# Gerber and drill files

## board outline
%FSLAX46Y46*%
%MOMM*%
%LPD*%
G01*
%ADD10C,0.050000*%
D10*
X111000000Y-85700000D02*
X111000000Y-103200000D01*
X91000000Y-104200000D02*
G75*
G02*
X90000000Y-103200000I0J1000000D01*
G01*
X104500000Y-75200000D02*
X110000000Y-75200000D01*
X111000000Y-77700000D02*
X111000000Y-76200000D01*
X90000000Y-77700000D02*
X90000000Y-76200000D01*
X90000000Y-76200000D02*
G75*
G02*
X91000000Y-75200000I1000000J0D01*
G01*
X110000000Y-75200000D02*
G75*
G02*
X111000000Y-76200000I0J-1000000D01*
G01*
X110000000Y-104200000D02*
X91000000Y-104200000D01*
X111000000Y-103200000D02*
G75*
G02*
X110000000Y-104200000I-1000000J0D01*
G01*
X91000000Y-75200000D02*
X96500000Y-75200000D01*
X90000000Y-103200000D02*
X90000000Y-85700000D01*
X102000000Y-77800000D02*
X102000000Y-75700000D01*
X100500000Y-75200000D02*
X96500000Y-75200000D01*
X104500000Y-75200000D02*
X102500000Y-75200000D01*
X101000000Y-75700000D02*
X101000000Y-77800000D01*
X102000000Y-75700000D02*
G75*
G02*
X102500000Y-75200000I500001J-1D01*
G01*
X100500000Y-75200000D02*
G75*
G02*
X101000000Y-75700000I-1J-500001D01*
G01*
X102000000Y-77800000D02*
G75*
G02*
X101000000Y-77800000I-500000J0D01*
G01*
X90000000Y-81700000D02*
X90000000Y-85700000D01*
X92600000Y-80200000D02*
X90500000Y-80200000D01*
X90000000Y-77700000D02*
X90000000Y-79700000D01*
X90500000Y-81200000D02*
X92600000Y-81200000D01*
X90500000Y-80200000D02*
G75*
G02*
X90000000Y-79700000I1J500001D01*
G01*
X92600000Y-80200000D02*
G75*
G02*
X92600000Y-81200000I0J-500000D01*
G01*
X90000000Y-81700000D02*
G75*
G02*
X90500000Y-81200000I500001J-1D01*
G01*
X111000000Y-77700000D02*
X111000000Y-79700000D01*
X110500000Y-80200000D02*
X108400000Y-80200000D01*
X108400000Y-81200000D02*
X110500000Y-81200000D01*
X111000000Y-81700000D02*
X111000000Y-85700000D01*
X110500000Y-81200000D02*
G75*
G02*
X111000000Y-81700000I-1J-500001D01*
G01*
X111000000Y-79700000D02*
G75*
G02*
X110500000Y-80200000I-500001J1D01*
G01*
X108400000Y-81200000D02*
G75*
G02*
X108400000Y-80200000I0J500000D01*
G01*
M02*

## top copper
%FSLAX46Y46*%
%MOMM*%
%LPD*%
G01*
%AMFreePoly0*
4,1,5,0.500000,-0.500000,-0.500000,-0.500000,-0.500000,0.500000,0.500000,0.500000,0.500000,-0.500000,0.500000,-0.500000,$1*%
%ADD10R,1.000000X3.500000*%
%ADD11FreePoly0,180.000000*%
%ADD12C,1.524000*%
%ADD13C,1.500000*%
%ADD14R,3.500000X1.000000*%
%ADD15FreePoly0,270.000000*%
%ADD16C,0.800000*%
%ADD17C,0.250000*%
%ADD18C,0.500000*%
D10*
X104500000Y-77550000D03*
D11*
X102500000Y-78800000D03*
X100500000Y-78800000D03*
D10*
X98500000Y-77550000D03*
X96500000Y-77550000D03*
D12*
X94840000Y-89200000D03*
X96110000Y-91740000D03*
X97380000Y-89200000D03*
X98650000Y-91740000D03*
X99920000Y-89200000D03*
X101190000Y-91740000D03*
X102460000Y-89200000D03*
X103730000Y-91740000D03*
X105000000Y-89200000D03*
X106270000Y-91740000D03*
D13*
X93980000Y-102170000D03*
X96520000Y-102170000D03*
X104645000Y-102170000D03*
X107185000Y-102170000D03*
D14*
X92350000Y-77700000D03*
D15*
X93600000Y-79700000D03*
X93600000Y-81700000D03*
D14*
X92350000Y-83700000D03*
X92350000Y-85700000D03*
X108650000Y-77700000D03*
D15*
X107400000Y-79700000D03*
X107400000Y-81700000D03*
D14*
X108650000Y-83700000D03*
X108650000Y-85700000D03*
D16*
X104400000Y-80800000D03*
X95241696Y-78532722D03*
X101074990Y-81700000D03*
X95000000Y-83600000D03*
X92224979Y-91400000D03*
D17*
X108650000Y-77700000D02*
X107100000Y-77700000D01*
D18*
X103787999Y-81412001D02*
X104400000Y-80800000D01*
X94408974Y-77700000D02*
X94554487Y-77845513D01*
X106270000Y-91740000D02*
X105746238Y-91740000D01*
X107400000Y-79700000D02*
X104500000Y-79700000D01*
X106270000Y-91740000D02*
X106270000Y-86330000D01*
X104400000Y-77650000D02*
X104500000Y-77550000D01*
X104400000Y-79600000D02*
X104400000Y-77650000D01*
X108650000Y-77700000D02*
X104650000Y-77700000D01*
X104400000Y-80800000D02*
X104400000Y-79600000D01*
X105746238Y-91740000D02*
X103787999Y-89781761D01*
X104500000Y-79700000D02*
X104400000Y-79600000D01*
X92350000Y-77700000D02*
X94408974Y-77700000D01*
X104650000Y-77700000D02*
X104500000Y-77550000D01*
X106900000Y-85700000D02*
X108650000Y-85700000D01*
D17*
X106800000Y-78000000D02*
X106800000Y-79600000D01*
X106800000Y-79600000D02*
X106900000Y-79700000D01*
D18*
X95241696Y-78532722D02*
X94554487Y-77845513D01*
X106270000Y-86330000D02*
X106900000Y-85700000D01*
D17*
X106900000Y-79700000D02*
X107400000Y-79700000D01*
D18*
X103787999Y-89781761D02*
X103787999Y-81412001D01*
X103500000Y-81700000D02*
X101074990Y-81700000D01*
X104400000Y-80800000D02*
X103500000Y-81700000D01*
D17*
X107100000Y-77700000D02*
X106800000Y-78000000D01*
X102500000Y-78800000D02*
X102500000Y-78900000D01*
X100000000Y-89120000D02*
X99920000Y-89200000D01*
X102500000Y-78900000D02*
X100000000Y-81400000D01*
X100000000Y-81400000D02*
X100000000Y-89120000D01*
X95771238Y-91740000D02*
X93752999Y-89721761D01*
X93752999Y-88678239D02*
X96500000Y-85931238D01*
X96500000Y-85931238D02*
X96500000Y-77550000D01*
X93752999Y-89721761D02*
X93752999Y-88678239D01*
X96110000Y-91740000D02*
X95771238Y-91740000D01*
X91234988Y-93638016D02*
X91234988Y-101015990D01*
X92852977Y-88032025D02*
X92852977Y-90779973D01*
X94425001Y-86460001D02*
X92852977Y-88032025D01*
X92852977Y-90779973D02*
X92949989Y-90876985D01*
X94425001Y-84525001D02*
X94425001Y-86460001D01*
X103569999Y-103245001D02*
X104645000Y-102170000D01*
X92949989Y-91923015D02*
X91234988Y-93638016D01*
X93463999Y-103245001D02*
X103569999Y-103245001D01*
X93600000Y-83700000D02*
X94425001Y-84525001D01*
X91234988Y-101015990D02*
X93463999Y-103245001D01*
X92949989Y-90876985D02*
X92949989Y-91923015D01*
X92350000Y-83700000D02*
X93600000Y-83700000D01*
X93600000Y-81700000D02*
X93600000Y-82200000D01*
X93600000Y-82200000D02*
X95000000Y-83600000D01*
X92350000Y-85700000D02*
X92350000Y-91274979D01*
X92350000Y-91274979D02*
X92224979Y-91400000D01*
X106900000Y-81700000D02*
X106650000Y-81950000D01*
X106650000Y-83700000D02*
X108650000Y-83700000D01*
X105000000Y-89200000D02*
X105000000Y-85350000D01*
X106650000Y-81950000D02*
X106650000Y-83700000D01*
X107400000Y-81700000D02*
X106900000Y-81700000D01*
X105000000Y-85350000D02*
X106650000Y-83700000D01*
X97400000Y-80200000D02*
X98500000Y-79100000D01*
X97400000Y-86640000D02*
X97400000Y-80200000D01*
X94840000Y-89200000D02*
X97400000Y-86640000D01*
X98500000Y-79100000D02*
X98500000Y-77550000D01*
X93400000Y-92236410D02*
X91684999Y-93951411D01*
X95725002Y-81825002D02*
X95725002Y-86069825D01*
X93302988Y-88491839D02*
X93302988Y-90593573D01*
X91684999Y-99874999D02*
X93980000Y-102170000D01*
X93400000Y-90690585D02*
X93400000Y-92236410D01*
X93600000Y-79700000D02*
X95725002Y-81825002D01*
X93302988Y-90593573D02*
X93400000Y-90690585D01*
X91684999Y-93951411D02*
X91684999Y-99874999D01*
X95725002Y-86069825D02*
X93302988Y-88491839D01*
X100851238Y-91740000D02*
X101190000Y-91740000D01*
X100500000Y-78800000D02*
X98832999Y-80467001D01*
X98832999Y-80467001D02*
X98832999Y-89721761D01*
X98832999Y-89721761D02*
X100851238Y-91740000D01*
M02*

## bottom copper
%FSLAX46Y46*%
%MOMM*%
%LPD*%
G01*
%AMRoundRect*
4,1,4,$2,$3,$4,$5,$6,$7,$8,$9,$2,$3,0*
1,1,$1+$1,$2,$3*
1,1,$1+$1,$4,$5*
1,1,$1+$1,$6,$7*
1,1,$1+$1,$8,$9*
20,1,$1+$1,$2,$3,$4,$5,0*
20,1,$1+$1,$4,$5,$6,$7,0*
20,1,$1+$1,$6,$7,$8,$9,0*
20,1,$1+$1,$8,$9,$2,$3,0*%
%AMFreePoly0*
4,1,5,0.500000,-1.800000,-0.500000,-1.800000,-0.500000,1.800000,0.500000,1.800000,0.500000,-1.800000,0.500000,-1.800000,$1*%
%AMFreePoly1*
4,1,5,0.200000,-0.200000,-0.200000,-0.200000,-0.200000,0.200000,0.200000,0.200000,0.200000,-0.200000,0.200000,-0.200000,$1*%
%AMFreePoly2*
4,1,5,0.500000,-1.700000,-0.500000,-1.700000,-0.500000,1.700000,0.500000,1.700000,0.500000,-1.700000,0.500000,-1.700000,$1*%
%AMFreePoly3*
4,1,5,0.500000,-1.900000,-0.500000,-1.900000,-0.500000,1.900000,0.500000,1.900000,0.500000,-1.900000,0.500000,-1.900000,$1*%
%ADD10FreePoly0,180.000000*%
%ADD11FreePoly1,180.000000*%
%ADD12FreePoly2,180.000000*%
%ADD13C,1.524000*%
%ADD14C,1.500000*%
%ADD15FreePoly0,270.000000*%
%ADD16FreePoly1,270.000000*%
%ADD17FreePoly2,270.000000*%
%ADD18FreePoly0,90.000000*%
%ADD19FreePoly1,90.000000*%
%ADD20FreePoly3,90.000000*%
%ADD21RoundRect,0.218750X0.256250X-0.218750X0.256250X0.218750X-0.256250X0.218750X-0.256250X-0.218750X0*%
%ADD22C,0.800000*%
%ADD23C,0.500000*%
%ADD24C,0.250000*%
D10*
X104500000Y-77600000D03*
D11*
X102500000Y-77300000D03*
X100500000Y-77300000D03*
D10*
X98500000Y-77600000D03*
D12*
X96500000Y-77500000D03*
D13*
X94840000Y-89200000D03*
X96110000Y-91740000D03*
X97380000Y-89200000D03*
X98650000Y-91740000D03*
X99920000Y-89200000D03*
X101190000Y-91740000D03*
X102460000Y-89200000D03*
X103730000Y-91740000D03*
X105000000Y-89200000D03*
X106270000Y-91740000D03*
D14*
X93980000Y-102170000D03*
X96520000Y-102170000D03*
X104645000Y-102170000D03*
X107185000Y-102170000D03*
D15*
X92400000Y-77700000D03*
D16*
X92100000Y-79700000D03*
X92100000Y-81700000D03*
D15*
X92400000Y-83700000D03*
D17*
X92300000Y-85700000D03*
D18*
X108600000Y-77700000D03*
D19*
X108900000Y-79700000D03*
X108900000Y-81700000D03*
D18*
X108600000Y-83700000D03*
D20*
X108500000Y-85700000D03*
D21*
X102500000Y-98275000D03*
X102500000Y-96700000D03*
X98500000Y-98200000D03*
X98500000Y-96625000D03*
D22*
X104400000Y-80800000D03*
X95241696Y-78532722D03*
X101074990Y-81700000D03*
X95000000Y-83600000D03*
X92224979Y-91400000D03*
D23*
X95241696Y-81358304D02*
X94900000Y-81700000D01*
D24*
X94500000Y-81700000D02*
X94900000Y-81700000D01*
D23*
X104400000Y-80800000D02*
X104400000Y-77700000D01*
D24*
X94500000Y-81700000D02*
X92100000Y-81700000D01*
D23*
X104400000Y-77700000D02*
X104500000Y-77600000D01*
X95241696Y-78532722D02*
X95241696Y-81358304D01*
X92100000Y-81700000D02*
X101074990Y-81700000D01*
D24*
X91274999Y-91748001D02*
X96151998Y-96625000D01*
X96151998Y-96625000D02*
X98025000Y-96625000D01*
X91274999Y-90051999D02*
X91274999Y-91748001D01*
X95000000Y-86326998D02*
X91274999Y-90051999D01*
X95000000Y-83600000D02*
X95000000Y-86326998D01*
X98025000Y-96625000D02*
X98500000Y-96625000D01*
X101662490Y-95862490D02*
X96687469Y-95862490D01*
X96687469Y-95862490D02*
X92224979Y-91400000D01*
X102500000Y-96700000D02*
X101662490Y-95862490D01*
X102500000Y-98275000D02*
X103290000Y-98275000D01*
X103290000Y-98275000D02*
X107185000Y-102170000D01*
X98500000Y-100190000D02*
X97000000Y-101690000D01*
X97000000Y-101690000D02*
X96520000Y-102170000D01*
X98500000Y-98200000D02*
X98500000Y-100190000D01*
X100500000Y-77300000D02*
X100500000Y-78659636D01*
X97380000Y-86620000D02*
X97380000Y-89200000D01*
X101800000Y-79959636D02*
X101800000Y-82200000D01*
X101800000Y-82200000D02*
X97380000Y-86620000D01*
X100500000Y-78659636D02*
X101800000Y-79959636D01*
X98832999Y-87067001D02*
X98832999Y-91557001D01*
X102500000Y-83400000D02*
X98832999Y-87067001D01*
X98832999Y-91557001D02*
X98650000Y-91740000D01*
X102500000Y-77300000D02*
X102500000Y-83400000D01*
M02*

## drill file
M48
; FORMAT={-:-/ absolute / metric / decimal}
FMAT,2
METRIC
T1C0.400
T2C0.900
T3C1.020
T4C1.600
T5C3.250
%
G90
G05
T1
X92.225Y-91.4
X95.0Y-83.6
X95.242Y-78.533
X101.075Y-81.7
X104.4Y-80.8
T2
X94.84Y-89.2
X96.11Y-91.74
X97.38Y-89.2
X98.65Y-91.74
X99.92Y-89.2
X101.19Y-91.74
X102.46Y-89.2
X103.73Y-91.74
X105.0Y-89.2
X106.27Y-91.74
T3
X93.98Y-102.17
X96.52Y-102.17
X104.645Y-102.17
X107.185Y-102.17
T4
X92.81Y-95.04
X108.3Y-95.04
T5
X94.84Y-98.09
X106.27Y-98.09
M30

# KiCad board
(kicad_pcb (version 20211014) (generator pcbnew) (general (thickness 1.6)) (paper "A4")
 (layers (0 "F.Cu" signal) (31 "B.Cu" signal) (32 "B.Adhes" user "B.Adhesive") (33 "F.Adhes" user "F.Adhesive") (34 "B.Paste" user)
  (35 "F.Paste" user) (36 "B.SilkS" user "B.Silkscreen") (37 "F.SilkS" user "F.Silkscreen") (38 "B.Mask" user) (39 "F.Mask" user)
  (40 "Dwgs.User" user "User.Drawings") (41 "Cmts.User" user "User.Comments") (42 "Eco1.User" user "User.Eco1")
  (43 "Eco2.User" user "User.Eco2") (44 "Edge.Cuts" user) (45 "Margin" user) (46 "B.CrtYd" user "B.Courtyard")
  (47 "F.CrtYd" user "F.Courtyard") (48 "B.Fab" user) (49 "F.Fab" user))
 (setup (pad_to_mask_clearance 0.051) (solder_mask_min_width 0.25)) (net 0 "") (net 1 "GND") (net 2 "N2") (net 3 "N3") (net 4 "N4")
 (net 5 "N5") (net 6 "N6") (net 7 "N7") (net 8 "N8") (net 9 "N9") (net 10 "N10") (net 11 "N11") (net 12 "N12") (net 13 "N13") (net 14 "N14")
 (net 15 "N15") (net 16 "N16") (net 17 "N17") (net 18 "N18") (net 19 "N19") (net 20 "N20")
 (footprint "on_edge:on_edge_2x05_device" (layer "F.Cu") (at 100.5 75.2 180)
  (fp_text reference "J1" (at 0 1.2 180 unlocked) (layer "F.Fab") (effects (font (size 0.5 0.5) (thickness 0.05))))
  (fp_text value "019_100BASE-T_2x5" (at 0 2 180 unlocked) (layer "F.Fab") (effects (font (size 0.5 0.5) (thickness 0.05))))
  (fp_line (start -1.5 -2.6) (end -1.5 -0.5) (layer "Edge.Cuts") (width 0.05))
  (fp_line (start 0 0) (end 4 0) (layer "Edge.Cuts") (width 0.05))
  (fp_line (start -4 0) (end -2 0) (layer "Edge.Cuts") (width 0.05))
  (fp_line (start -0.5 -0.5) (end -0.5 -2.6) (layer "Edge.Cuts") (width 0.05))
  (fp_arc (start -1.5 -0.5) (mid -1.646447 -0.146447) (end -2 0) (layer "Edge.Cuts") (width 0.05))
  (fp_arc (start 0 0) (mid -0.353553 -0.146447) (end -0.5 -0.5) (layer "Edge.Cuts") (width 0.05))
  (fp_arc (start -1.5 -2.6) (mid -1 -3.1) (end -0.5 -2.6) (layer "Edge.Cuts") (width 0.05))
  (pad "1" smd rect locked (at -4 -2.35) (size 1 3.5) (layers "F.Cu" "F.Mask") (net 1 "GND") (zone_connect 0))
  (pad "2" smd custom locked (at -2 -3.6 180) (size 1 1) (layers "F.Cu" "F.Mask") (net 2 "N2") (zone_connect 0)
   (options (clearance outline) (anchor rect)) (primitives))
  (pad "3" smd custom locked (at 0 -3.6 180) (size 1 1) (layers "F.Cu" "F.Mask") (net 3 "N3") (zone_connect 0)
   (options (clearance outline) (anchor rect)) (primitives))
  (pad "4" smd rect locked (at 2 -2.35) (size 1 3.5) (layers "F.Cu" "F.Mask") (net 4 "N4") (zone_connect 0))
  (pad "5" smd rect locked (at 4 -2.35) (size 1 3.5) (layers "F.Cu" "F.Mask") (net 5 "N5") (zone_connect 0))
  (pad "6" smd custom locked (at -4 -2.4 180) (size 1 3.6) (layers "B.Cu" "B.Mask") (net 1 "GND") (zone_connect 0)
   (options (clearance outline) (anchor rect)) (primitives))
  (pad "7" smd custom locked (at -2 -2.1 180) (size 0.4 0.4) (layers "B.Cu" "B.Mask") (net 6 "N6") (zone_connect 0)
   (options (clearance outline) (anchor rect)) (primitives))
  (pad "8" smd custom locked (at 0 -2.1 180) (size 0.4 0.4) (layers "B.Cu" "B.Mask") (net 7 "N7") (zone_connect 0)
   (options (clearance outline) (anchor rect)) (primitives))
  (pad "9" smd custom locked (at 2 -2.4 180) (size 1 3.6) (layers "B.Cu" "B.Mask") (zone_connect 0)
   (options (clearance outline) (anchor rect)) (primitives))
  (pad "10" smd custom locked (at 4 -2.3 180) (size 1 3.4) (layers "B.Cu" "B.Mask") (zone_connect 0)
   (options (clearance outline) (anchor rect)) (primitives)))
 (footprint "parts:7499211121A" (layer "F.Cu") (at 105 89.2 180)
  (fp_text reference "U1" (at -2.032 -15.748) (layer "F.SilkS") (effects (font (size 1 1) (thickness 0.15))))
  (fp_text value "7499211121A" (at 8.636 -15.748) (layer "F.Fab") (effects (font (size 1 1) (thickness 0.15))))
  (pad "" np_thru_hole circle (at -3.3 -5.84 180) (size 1.6 1.6) (drill 1.6) (layers *.Cu *.Mask))
  (pad "" np_thru_hole circle (at 10.16 -8.89 180) (size 3.25 3.25) (drill 3.25) (layers *.Cu *.Mask))
  (pad "" np_thru_hole circle (at 12.19 -5.84 180) (size 1.6 1.6) (drill 1.6) (layers *.Cu *.Mask))
  (pad "" np_thru_hole circle (at -1.27 -8.89 180) (size 3.25 3.25) (drill 3.25) (layers *.Cu *.Mask))
  (pad "1" thru_hole circle (at 10.16 0 180) (size 1.524 1.524) (drill 0.9) (layers *.Cu *.Mask) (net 4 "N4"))
  (pad "2" thru_hole circle (at 8.89 -2.54 180) (size 1.524 1.524) (drill 0.9) (layers *.Cu *.Mask) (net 5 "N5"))
  (pad "3" thru_hole circle (at 7.62 0 180) (size 1.524 1.524) (drill 0.9) (layers *.Cu *.Mask) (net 7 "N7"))
  (pad "4" thru_hole circle (at 6.35 -2.54 180) (size 1.524 1.524) (drill 0.9) (layers *.Cu *.Mask) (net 6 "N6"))
  (pad "5" thru_hole circle (at 5.08 0 180) (size 1.524 1.524) (drill 0.9) (layers *.Cu *.Mask) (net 2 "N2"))
  (pad "6" thru_hole circle (at 3.81 -2.54 180) (size 1.524 1.524) (drill 0.9) (layers *.Cu *.Mask) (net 3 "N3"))
  (pad "7" thru_hole circle (at 2.54 0 180) (size 1.524 1.524) (drill 0.9) (layers *.Cu *.Mask) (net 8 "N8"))
  (pad "8" thru_hole circle (at 1.27 -2.54 180) (size 1.524 1.524) (drill 0.9) (layers *.Cu *.Mask) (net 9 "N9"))
  (pad "9" thru_hole circle (at 0 0 180) (size 1.524 1.524) (drill 0.9) (layers *.Cu *.Mask) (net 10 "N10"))
  (pad "10" thru_hole circle (at -1.27 -2.54 180) (size 1.524 1.524) (drill 0.9) (layers *.Cu *.Mask) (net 1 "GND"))
  (pad "11" thru_hole circle (at 11.02 -12.97 180) (size 1.5 1.5) (drill 1.02) (layers *.Cu *.Mask) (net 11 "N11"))
  (pad "12" thru_hole circle (at 8.48 -12.97 180) (size 1.5 1.5) (drill 1.02) (layers *.Cu *.Mask) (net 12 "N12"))
  (pad "13" thru_hole circle (at 0.355 -12.97 180) (size 1.5 1.5) (drill 1.02) (layers *.Cu *.Mask) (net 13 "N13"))
  (pad "14" thru_hole circle (at -2.185 -12.97 180) (size 1.5 1.5) (drill 1.02) (layers *.Cu *.Mask) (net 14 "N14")))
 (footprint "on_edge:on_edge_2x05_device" (layer "F.Cu") (at 90 81.7 -90)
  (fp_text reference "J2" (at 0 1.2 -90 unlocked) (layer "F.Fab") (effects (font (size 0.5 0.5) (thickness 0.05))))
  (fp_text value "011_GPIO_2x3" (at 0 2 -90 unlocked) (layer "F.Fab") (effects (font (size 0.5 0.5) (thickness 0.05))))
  (fp_line (start 0 0) (end 4 0) (layer "Edge.Cuts") (width 0.05))
  (fp_line (start -1.5 -2.6) (end -1.5 -0.5) (layer "Edge.Cuts") (width 0.05))
  (fp_line (start -4 0) (end -2 0) (layer "Edge.Cuts") (width 0.05))
  (fp_line (start -0.5 -0.5) (end -0.5 -2.6) (layer "Edge.Cuts") (width 0.05))
  (fp_arc (start -1.5 -0.5) (mid -1.646447 -0.146447) (end -2 0) (layer "Edge.Cuts") (width 0.05))
  (fp_arc (start -1.5 -2.6) (mid -1 -3.1) (end -0.5 -2.6) (layer "Edge.Cuts") (width 0.05))
  (fp_arc (start 0 0) (mid -0.353553 -0.146447) (end -0.5 -0.5) (layer "Edge.Cuts") (width 0.05))
  (pad "1" smd rect locked (at -4 -2.35 90) (size 1 3.5) (layers "F.Cu" "F.Mask") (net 1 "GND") (zone_connect 0))
  (pad "2" smd custom locked (at -2 -3.6 270) (size 1 1) (layers "F.Cu" "F.Mask") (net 11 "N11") (zone_connect 0)
   (options (clearance outline) (anchor rect)) (primitives))
  (pad "3" smd custom locked (at 0 -3.6 270) (size 1 1) (layers "F.Cu" "F.Mask") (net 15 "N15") (zone_connect 0)
   (options (clearance outline) (anchor rect)) (primitives))
  (pad "4" smd rect locked (at 2 -2.35 90) (size 1 3.5) (layers "F.Cu" "F.Mask") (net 13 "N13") (zone_connect 0))
  (pad "5" smd rect locked (at 4 -2.35 90) (size 1 3.5) (layers "F.Cu" "F.Mask") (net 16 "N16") (zone_connect 0))
  (pad "6" smd custom locked (at -4 -2.4 270) (size 1 3.6) (layers "B.Cu" "B.Mask") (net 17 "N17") (zone_connect 0)
   (options (clearance outline) (anchor rect)) (primitives))
  (pad "7" smd custom locked (at -2 -2.1 270) (size 0.4 0.4) (layers "B.Cu" "B.Mask") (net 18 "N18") (zone_connect 0)
   (options (clearance outline) (anchor rect)) (primitives))
  (pad "8" smd custom locked (at 0 -2.1 270) (size 0.4 0.4) (layers "B.Cu" "B.Mask") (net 1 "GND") (zone_connect 0)
   (options (clearance outline) (anchor rect)) (primitives))
  (pad "9" smd custom locked (at 2 -2.4 270) (size 1 3.6) (layers "B.Cu" "B.Mask") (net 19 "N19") (zone_connect 0)
   (options (clearance outline) (anchor rect)) (primitives))
  (pad "10" smd custom locked (at 4 -2.3 270) (size 1 3.4) (layers "B.Cu" "B.Mask") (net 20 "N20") (zone_connect 0)
   (options (clearance outline) (anchor rect)) (primitives)))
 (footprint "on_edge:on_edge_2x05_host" (layer "F.Cu") (at 111 81.7 -90)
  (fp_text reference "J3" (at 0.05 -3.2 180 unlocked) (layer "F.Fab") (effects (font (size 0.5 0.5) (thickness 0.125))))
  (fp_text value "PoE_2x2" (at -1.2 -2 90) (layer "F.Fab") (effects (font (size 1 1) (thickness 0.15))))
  (fp_line (start -4 0) (end -2 0) (layer "Edge.Cuts") (width 0.05))
  (fp_line (start -1.5 0.5) (end -1.5 2.6) (layer "Edge.Cuts") (width 0.05))
  (fp_line (start -0.5 2.6) (end -0.5 0.5) (layer "Edge.Cuts") (width 0.05))
  (fp_line (start 0 0) (end 4 0) (layer "Edge.Cuts") (width 0.05))
  (fp_arc (start -0.5 0.5) (mid -0.353553 0.146447) (end 0 0) (layer "Edge.Cuts") (width 0.05))
  (fp_arc (start -2 0) (mid -1.646447 0.146447) (end -1.5 0.5) (layer "Edge.Cuts") (width 0.05))
  (fp_arc (start -0.5 2.6) (mid -1 3.1) (end -1.5 2.6) (layer "Edge.Cuts") (width 0.05))
  (pad "1" smd rect locked (at -4 2.35 270) (size 1 3.5) (layers "F.Cu" "F.Mask") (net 1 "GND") (zone_connect 0))
  (pad "2" smd custom locked (at -2 3.6 270) (size 1 1) (layers "F.Cu" "F.Mask") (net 1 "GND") (zone_connect 0)
   (options (clearance outline) (anchor rect)) (primitives))
  (pad "3" smd custom locked (at 0 3.6 270) (size 1 1) (layers "F.Cu" "F.Mask") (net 10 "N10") (zone_connect 0)
   (options (clearance outline) (anchor rect)) (primitives))
  (pad "4" smd rect locked (at 2 2.35 270) (size 1 3.5) (layers "F.Cu" "F.Mask") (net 10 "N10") (zone_connect 0))
  (pad "5" smd rect locked (at 4 2.35 270) (size 1 3.5) (layers "F.Cu" "F.Mask") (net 1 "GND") (zone_connect 0))
  (pad "6" smd custom locked (at -4 2.4 90) (size 1 3.6) (layers "B.Cu" "B.Mask") (zone_connect 0)
   (options (clearance outline) (anchor rect)) (primitives))
  (pad "7" smd custom locked (at -2 2.1 90) (size 0.4 0.4) (layers "B.Cu" "B.Mask") (zone_connect 0)
   (options (clearance outline) (anchor rect)) (primitives))
  (pad "8" smd custom locked (at 0 2.1 90) (size 0.4 0.4) (layers "B.Cu" "B.Mask") (zone_connect 0)
   (options (clearance outline) (anchor rect)) (primitives))
  (pad "9" smd custom locked (at 2 2.4 90) (size 1 3.6) (layers "B.Cu" "B.Mask") (zone_connect 0)
   (options (clearance outline) (anchor rect)) (primitives))
  (pad "10" smd custom locked (at 4 2.5 90) (size 1 3.8) (layers "B.Cu" "B.Mask") (zone_connect 0)
   (options (clearance outline) (anchor rect)) (primitives)))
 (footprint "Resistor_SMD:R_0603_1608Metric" (layer "B.Cu") (at 102.5 97.4875 90)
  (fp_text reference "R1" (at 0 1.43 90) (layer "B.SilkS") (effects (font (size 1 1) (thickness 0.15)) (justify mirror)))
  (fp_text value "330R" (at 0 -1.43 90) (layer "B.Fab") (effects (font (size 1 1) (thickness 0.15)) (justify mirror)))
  (pad "1" smd roundrect locked (at -0.7875 0 90) (size 0.875 0.95) (layers "B.Cu" "B.Paste" "B.Mask") (roundrect_rratio 0.25)
   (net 14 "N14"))
  (pad "2" smd roundrect locked (at 0.7875 0 90) (size 0.875 0.95) (layers "B.Cu" "B.Paste" "B.Mask") (roundrect_rratio 0.25) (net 16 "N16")))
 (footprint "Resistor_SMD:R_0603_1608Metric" (layer "B.Cu") (at 98.5 97.4125 90)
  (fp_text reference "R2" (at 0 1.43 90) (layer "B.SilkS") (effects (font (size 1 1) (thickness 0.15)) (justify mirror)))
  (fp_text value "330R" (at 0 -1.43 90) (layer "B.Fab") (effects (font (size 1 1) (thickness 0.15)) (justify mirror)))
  (pad "1" smd roundrect locked (at -0.7875 0 90) (size 0.875 0.95) (layers "B.Cu" "B.Paste" "B.Mask") (roundrect_rratio 0.25)
   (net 12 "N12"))
  (pad "2" smd roundrect locked (at 0.7875 0 90) (size 0.875 0.95) (layers "B.Cu" "B.Paste" "B.Mask") (roundrect_rratio 0.25) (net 15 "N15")))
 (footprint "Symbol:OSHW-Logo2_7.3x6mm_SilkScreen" (layer "B.Cu") (at 100.2 83.6 180)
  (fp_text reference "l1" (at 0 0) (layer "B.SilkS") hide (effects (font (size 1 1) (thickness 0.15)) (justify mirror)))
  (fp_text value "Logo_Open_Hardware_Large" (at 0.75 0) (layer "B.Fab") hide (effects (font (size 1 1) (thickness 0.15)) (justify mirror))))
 (gr_line (start 111 85.7) (end 111 103.2) (layer "Edge.Cuts") (width 0.05))
 (gr_arc (start 91 104.2) (mid 90.292893 103.907107) (end 90 103.2) (layer "Edge.Cuts") (width 0.05))
 (gr_line (start 104.5 75.2) (end 110 75.2) (layer "Edge.Cuts") (width 0.05))
 (gr_line (start 111 77.7) (end 111 76.2) (layer "Edge.Cuts") (width 0.05))
 (gr_line (start 90 77.7) (end 90 76.2) (layer "Edge.Cuts") (width 0.05))
 (gr_arc (start 90 76.2) (mid 90.292893 75.492893) (end 91 75.2) (layer "Edge.Cuts") (width 0.05))
 (gr_arc (start 110 75.2) (mid 110.707107 75.492893) (end 111 76.2) (layer "Edge.Cuts") (width 0.05))
 (gr_line (start 110 104.2) (end 91 104.2) (layer "Edge.Cuts") (width 0.05))
 (gr_arc (start 111 103.2) (mid 110.707107 103.907107) (end 110 104.2) (layer "Edge.Cuts") (width 0.05))
 (gr_line (start 91 75.2) (end 96.5 75.2) (layer "Edge.Cuts") (width 0.05))
 (gr_line (start 90 103.2) (end 90 85.7) (layer "Edge.Cuts") (width 0.05))
 (segment (start 108.65 77.7) (end 107.1 77.7) (width 0.25) (layer "F.Cu") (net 1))
 (segment (start 103.787999 81.412001) (end 104.4 80.8) (width 0.5) (layer "F.Cu") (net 1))
 (segment (start 94.408974 77.7) (end 94.554487 77.845513) (width 0.5) (layer "F.Cu") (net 1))
 (segment (start 106.27 91.74) (end 105.746238 91.74) (width 0.5) (layer "F.Cu") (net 1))
 (segment (start 107.4 79.7) (end 104.5 79.7) (width 0.5) (layer "F.Cu") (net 1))
 (segment (start 106.27 91.74) (end 106.27 86.33) (width 0.5) (layer "F.Cu") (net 1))
 (segment (start 104.4 77.65) (end 104.5 77.55) (width 0.5) (layer "F.Cu") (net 1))
 (segment (start 104.4 79.6) (end 104.4 77.65) (width 0.5) (layer "F.Cu") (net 1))
 (segment (start 108.65 77.7) (end 104.65 77.7) (width 0.5) (layer "F.Cu") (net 1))
 (segment (start 104.4 80.8) (end 104.4 79.6) (width 0.5) (layer "F.Cu") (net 1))
 (segment (start 105.746238 91.74) (end 103.787999 89.781761) (width 0.5) (layer "F.Cu") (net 1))
 (segment (start 104.5 79.7) (end 104.4 79.6) (width 0.5) (layer "F.Cu") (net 1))
 (segment (start 92.35 77.7) (end 94.408974 77.7) (width 0.5) (layer "F.Cu") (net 1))
 (segment (start 104.65 77.7) (end 104.5 77.55) (width 0.5) (layer "F.Cu") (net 1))
 (segment (start 106.9 85.7) (end 108.65 85.7) (width 0.5) (layer "F.Cu") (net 1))
 (segment (start 106.8 78) (end 106.8 79.6) (width 0.25) (layer "F.Cu") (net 1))
 (segment (start 106.8 79.6) (end 106.9 79.7) (width 0.25) (layer "F.Cu") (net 1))
 (segment (start 95.241696 78.532722) (end 94.554487 77.845513) (width 0.5) (layer "F.Cu") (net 1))
 (segment (start 106.27 86.33) (end 106.9 85.7) (width 0.5) (layer "F.Cu") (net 1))
 (segment (start 106.9 79.7) (end 107.4 79.7) (width 0.25) (layer "F.Cu") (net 1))
 (segment (start 103.787999 89.781761) (end 103.787999 81.412001) (width 0.5) (layer "F.Cu") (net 1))
 (segment (start 103.5 81.7) (end 101.07499 81.7) (width 0.5) (layer "F.Cu") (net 1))
 (segment (start 104.4 80.8) (end 103.5 81.7) (width 0.5) (layer "F.Cu") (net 1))
 (segment (start 107.1 77.7) (end 106.8 78) (width 0.25) (layer "F.Cu") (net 1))
 (via (at 104.4 80.8) (size 0.8) (drill 0.4) (layers "F.Cu" "B.Cu") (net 1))
 (via (at 95.241696 78.532722) (size 0.8) (drill 0.4) (layers "F.Cu" "B.Cu") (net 1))
 (via (at 101.07499 81.7) (size 0.8) (drill 0.4) (layers "F.Cu" "B.Cu") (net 1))
 (segment (start 95.241696 81.358304) (end 94.9 81.7) (width 0.5) (layer "B.Cu") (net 1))
 (segment (start 94.5 81.7) (end 94.9 81.7) (width 0.25) (layer "B.Cu") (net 1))
 (segment (start 104.4 80.8) (end 104.4 77.7) (width 0.5) (layer "B.Cu") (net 1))
 (segment (start 94.5 81.7) (end 92.1 81.7) (width 0.25) (layer "B.Cu") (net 1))
 (segment (start 104.4 77.7) (end 104.5 77.6) (width 0.5) (layer "B.Cu") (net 1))
 (segment (start 95.241696 78.532722) (end 95.241696 81.358304) (width 0.5) (layer "B.Cu") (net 1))
 (segment (start 92.1 81.7) (end 101.07499 81.7) (width 0.5) (layer "B.Cu") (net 1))
 (segment (start 102.5 78.8) (end 102.5 78.9) (width 0.25) (layer "F.Cu") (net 2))
 (segment (start 100 89.12) (end 99.92 89.2) (width 0.25) (layer "F.Cu") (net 2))
 (segment (start 102.5 78.9) (end 100 81.4) (width 0.25) (layer "F.Cu") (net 2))
 (segment (start 100 81.4) (end 100 89.12) (width 0.25) (layer "F.Cu") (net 2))
 (segment (start 95.771238 91.74) (end 93.752999 89.721761) (width 0.25) (layer "F.Cu") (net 5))
 (segment (start 93.752999 88.678239) (end 96.5 85.931238) (width 0.25) (layer "F.Cu") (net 5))
 (segment (start 96.5 85.931238) (end 96.5 77.55) (width 0.25) (layer "F.Cu") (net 5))
 (segment (start 93.752999 89.721761) (end 93.752999 88.678239) (width 0.25) (layer "F.Cu") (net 5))
 (segment (start 96.11 91.74) (end 95.771238 91.74) (width 0.25) (layer "F.Cu") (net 5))
 (segment (start 91.234988 93.638016) (end 91.234988 101.01599) (width 0.25) (layer "F.Cu") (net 13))
 (segment (start 92.852977 88.032025) (end 92.852977 90.779973) (width 0.25) (layer "F.Cu") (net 13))
 (segment (start 94.425001 86.460001) (end 92.852977 88.032025) (width 0.25) (layer "F.Cu") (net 13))
 (segment (start 92.852977 90.779973) (end 92.949989 90.876985) (width 0.25) (layer "F.Cu") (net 13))
 (segment (start 94.425001 84.525001) (end 94.425001 86.460001) (width 0.25) (layer "F.Cu") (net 13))
 (segment (start 103.569999 103.245001) (end 104.645 102.17) (width 0.25) (layer "F.Cu") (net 13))
 (segment (start 92.949989 91.923015) (end 91.234988 93.638016) (width 0.25) (layer "F.Cu") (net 13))
 (segment (start 93.463999 103.245001) (end 103.569999 103.245001) (width 0.25) (layer "F.Cu") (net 13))
 (segment (start 93.6 83.7) (end 94.425001 84.525001) (width 0.25) (layer "F.Cu") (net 13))
 (segment (start 91.234988 101.01599) (end 93.463999 103.245001) (width 0.25) (layer "F.Cu") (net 13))
 (segment (start 92.949989 90.876985) (end 92.949989 91.923015) (width 0.25) (layer "F.Cu") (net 13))
 (segment (start 92.35 83.7) (end 93.6 83.7) (width 0.25) (layer "F.Cu") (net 13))
 (segment (start 93.6 81.7) (end 93.6 82.2) (width 0.25) (layer "F.Cu") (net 15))
 (segment (start 93.6 82.2) (end 95 83.6) (width 0.25) (layer "F.Cu") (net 15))
 (via (at 95 83.6) (size 0.8) (drill 0.4) (layers "F.Cu" "B.Cu") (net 15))
 (segment (start 91.274999 91.748001) (end 96.151998 96.625) (width 0.25) (layer "B.Cu") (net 15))
 (segment (start 96.151998 96.625) (end 98.025 96.625) (width 0.25) (layer "B.Cu") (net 15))
 (segment (start 91.274999 90.051999) (end 91.274999 91.748001) (width 0.25) (layer "B.Cu") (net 15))
 (segment (start 95 86.326998) (end 91.274999 90.051999) (width 0.25) (layer "B.Cu") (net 15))
 (segment (start 95 83.6) (end 95 86.326998) (width 0.25) (layer "B.Cu") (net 15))
 (segment (start 98.025 96.625) (end 98.5 96.625) (width 0.25) (layer "B.Cu") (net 15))
 (segment (start 92.35 85.7) (end 92.35 91.274979) (width 0.25) (layer "F.Cu") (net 16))
 (segment (start 92.35 91.274979) (end 92.224979 91.4) (width 0.25) (layer "F.Cu") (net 16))
 (via (at 92.224979 91.4) (size 0.8) (drill 0.4) (layers "F.Cu" "B.Cu") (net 16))
 (segment (start 101.66249 95.86249) (end 96.687469 95.86249) (width 0.25) (layer "B.Cu") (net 16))
 (segment (start 96.687469 95.86249) (end 92.224979 91.4) (width 0.25) (layer "B.Cu") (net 16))
 (segment (start 102.5 96.7) (end 101.66249 95.86249) (width 0.25) (layer "B.Cu") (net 16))
 (segment (start 106.9 81.7) (end 106.65 81.95) (width 0.25) (layer "F.Cu") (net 10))
 (segment (start 106.65 83.7) (end 108.65 83.7) (width 0.25) (layer "F.Cu") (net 10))
 (segment (start 105 89.2) (end 105 85.35) (width 0.25) (layer "F.Cu") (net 10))
 (segment (start 106.65 81.95) (end 106.65 83.7) (width 0.25) (layer "F.Cu") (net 10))
 (segment (start 107.4 81.7) (end 106.9 81.7) (width 0.25) (layer "F.Cu") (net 10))
 (segment (start 105 85.35) (end 106.65 83.7) (width 0.25) (layer "F.Cu") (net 10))
 (segment (start 102.5 98.275) (end 103.29 98.275) (width 0.25) (layer "B.Cu") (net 14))
 (segment (start 103.29 98.275) (end 107.185 102.17) (width 0.25) (layer "B.Cu") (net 14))
 (segment (start 98.5 100.19) (end 97 101.69) (width 0.25) (layer "B.Cu") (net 12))
 (segment (start 97 101.69) (end 96.52 102.17) (width 0.25) (layer "B.Cu") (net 12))
 (segment (start 98.5 98.2) (end 98.5 100.19) (width 0.25) (layer "B.Cu") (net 12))
 (segment (start 97.4 80.2) (end 98.5 79.1) (width 0.25) (layer "F.Cu") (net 4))
 (segment (start 97.4 86.64) (end 97.4 80.2) (width 0.25) (layer "F.Cu") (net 4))
 (segment (start 94.84 89.2) (end 97.4 86.64) (width 0.25) (layer "F.Cu") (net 4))
 (segment (start 98.5 79.1) (end 98.5 77.55) (width 0.25) (layer "F.Cu") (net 4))
 (segment (start 93.4 92.23641) (end 91.684999 93.951411) (width 0.25) (layer "F.Cu") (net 11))
 (segment (start 95.725002 81.825002) (end 95.725002 86.069825) (width 0.25) (layer "F.Cu") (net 11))
 (segment (start 93.302988 88.491839) (end 93.302988 90.593573) (width 0.25) (layer "F.Cu") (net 11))
 (segment (start 91.684999 99.874999) (end 93.98 102.17) (width 0.25) (layer "F.Cu") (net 11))
 (segment (start 93.4 90.690585) (end 93.4 92.23641) (width 0.25) (layer "F.Cu") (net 11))
 (segment (start 93.6 79.7) (end 95.725002 81.825002) (width 0.25) (layer "F.Cu") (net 11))
 (segment (start 93.302988 90.593573) (end 93.4 90.690585) (width 0.25) (layer "F.Cu") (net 11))
 (segment (start 91.684999 93.951411) (end 91.684999 99.874999) (width 0.25) (layer "F.Cu") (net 11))
 (segment (start 95.725002 86.069825) (end 93.302988 88.491839) (width 0.25) (layer "F.Cu") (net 11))
 (segment (start 100.851238 91.74) (end 101.19 91.74) (width 0.25) (layer "F.Cu") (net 3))
 (segment (start 100.5 78.8) (end 98.832999 80.467001) (width 0.25) (layer "F.Cu") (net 3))
 (segment (start 98.832999 80.467001) (end 98.832999 89.721761) (width 0.25) (layer "F.Cu") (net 3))
 (segment (start 98.832999 89.721761) (end 100.851238 91.74) (width 0.25) (layer "F.Cu") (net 3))
 (segment (start 100.5 77.3) (end 100.5 78.659636) (width 0.25) (layer "B.Cu") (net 7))
 (segment (start 97.38 86.62) (end 97.38 89.2) (width 0.25) (layer "B.Cu") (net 7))
 (segment (start 101.8 79.959636) (end 101.8 82.2) (width 0.25) (layer "B.Cu") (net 7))
 (segment (start 101.8 82.2) (end 97.38 86.62) (width 0.25) (layer "B.Cu") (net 7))
 (segment (start 100.5 78.659636) (end 101.8 79.959636) (width 0.25) (layer "B.Cu") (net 7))
 (segment (start 98.832999 87.067001) (end 98.832999 91.557001) (width 0.25) (layer "B.Cu") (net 6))
 (segment (start 102.5 83.4) (end 98.832999 87.067001) (width 0.25) (layer "B.Cu") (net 6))
 (segment (start 98.832999 91.557001) (end 98.65 91.74) (width 0.25) (layer "B.Cu") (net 6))
 (segment (start 102.5 77.3) (end 102.5 83.4) (width 0.25) (layer "B.Cu") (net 6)))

